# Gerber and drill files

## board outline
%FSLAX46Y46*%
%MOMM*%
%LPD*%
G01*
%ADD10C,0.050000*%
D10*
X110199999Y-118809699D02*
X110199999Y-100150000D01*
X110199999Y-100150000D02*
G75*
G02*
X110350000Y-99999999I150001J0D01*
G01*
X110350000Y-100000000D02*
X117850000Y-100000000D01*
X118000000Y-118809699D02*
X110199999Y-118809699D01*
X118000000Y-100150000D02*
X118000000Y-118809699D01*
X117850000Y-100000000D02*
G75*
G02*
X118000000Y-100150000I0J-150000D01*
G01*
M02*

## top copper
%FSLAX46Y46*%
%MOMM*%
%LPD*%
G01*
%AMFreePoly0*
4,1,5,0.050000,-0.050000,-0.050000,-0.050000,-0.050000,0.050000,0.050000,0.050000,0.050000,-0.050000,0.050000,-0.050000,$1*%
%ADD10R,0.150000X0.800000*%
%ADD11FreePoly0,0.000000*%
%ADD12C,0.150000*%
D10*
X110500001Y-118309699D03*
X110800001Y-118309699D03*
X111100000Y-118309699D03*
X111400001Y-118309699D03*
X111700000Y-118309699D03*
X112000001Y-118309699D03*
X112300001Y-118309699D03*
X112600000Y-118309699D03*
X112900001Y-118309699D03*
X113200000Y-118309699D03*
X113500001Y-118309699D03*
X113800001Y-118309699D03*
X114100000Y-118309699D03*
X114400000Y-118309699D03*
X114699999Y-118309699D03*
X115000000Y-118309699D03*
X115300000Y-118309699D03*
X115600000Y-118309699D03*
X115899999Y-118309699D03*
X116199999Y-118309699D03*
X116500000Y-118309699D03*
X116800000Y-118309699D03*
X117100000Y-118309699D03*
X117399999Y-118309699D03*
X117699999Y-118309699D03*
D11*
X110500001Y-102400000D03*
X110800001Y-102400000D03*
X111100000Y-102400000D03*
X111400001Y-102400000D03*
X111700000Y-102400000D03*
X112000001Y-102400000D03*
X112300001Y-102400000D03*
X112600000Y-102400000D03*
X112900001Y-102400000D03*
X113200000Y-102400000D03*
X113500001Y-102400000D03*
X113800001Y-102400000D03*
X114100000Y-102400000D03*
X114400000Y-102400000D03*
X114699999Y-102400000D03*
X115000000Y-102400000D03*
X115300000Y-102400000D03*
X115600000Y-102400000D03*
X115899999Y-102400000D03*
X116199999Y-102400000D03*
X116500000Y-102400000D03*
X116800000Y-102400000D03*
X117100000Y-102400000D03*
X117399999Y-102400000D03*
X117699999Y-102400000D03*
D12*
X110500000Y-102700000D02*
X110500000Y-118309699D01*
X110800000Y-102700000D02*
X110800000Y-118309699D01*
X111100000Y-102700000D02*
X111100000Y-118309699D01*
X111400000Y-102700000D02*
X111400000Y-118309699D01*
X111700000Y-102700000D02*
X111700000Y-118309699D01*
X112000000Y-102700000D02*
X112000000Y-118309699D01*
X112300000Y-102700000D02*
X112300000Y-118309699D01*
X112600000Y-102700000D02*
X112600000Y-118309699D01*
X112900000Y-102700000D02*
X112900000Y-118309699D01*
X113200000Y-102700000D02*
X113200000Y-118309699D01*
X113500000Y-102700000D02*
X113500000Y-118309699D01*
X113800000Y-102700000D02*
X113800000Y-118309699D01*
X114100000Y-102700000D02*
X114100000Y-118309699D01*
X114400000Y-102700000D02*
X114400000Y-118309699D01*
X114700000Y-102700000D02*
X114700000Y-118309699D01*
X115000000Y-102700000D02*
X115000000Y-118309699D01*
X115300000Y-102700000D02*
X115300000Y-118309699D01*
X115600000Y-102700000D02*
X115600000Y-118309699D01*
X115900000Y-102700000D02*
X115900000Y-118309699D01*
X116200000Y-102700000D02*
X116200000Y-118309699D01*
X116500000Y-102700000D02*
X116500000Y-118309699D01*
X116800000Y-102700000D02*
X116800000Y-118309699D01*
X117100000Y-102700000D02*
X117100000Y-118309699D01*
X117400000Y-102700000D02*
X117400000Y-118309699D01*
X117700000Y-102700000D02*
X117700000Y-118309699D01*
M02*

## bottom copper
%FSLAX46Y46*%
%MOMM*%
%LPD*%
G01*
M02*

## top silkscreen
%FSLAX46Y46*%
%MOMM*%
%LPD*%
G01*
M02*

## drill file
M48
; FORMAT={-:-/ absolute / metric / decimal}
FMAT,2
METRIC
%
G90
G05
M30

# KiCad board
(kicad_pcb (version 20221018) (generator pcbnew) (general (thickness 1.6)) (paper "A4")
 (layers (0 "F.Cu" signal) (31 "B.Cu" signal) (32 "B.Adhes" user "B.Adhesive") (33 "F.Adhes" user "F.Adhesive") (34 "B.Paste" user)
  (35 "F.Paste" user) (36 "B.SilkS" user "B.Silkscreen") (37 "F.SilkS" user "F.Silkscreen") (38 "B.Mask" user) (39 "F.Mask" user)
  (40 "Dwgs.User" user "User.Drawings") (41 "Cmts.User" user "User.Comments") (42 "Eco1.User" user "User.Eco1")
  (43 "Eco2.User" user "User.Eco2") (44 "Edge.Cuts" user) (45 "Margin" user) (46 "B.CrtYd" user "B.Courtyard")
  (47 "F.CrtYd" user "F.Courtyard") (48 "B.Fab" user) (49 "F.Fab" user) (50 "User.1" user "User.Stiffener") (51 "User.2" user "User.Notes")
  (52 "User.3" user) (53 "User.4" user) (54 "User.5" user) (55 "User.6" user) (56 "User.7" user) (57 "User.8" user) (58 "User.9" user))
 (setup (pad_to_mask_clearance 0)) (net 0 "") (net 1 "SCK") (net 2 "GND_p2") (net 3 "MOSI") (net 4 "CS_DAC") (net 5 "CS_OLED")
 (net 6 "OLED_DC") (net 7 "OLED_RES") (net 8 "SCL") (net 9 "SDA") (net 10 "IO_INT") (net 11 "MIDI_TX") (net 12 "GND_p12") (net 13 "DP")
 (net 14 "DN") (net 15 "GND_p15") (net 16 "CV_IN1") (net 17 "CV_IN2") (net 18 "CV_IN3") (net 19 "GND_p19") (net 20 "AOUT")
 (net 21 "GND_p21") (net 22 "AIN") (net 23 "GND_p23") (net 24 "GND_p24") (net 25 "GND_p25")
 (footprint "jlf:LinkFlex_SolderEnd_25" (layer "F.Cu") (at 114.1 118.809699)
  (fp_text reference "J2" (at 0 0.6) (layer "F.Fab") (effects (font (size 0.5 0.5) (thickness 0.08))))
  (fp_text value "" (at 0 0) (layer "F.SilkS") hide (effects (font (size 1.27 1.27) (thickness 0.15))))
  (pad "1" smd rect (at -3.599999 -0.5) (size 0.15 0.8) (layers "F.Cu" "F.Mask") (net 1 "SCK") (thermal_bridge_angle 45))
  (pad "2" smd rect (at -3.299999 -0.5) (size 0.15 0.8) (layers "F.Cu" "F.Mask") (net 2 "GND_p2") (thermal_bridge_angle 45))
  (pad "3" smd rect (at -3 -0.5) (size 0.15 0.8) (layers "F.Cu" "F.Mask") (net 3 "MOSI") (thermal_bridge_angle 45))
  (pad "4" smd rect (at -2.699999 -0.5) (size 0.15 0.8) (layers "F.Cu" "F.Mask") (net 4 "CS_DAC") (thermal_bridge_angle 45))
  (pad "5" smd rect (at -2.4 -0.5) (size 0.15 0.8) (layers "F.Cu" "F.Mask") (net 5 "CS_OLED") (thermal_bridge_angle 45))
  (pad "6" smd rect (at -2.099999 -0.5) (size 0.15 0.8) (layers "F.Cu" "F.Mask") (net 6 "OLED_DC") (thermal_bridge_angle 45))
  (pad "7" smd rect (at -1.799999 -0.5) (size 0.15 0.8) (layers "F.Cu" "F.Mask") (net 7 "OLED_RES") (thermal_bridge_angle 45))
  (pad "8" smd rect (at -1.5 -0.5) (size 0.15 0.8) (layers "F.Cu" "F.Mask") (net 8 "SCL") (thermal_bridge_angle 45))
  (pad "9" smd rect (at -1.199999 -0.5) (size 0.15 0.8) (layers "F.Cu" "F.Mask") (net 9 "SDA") (thermal_bridge_angle 45))
  (pad "10" smd rect (at -0.9 -0.5) (size 0.15 0.8) (layers "F.Cu" "F.Mask") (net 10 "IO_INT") (thermal_bridge_angle 45))
  (pad "11" smd rect (at -0.599999 -0.5) (size 0.15 0.8) (layers "F.Cu" "F.Mask") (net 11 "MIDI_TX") (thermal_bridge_angle 45))
  (pad "12" smd rect (at -0.299999 -0.5) (size 0.15 0.8) (layers "F.Cu" "F.Mask") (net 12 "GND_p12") (thermal_bridge_angle 45))
  (pad "13" smd rect (at 0 -0.5) (size 0.15 0.8) (layers "F.Cu" "F.Mask") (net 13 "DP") (thermal_bridge_angle 45))
  (pad "14" smd rect (at 0.3 -0.5) (size 0.15 0.8) (layers "F.Cu" "F.Mask") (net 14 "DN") (thermal_bridge_angle 45))
  (pad "15" smd rect (at 0.599999 -0.5) (size 0.15 0.8) (layers "F.Cu" "F.Mask") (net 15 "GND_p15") (thermal_bridge_angle 45))
  (pad "16" smd rect (at 0.9 -0.5) (size 0.15 0.8) (layers "F.Cu" "F.Mask") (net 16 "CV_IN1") (thermal_bridge_angle 45))
  (pad "17" smd rect (at 1.2 -0.5) (size 0.15 0.8) (layers "F.Cu" "F.Mask") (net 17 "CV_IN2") (thermal_bridge_angle 45))
  (pad "18" smd rect (at 1.5 -0.5) (size 0.15 0.8) (layers "F.Cu" "F.Mask") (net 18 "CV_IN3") (thermal_bridge_angle 45))
  (pad "19" smd rect (at 1.799999 -0.5) (size 0.15 0.8) (layers "F.Cu" "F.Mask") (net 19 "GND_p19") (thermal_bridge_angle 45))
  (pad "20" smd rect (at 2.099999 -0.5) (size 0.15 0.8) (layers "F.Cu" "F.Mask") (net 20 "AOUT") (thermal_bridge_angle 45))
  (pad "21" smd rect (at 2.4 -0.5) (size 0.15 0.8) (layers "F.Cu" "F.Mask") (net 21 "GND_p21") (thermal_bridge_angle 45))
  (pad "22" smd rect (at 2.7 -0.5) (size 0.15 0.8) (layers "F.Cu" "F.Mask") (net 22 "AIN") (thermal_bridge_angle 45))
  (pad "23" smd rect (at 3 -0.5) (size 0.15 0.8) (layers "F.Cu" "F.Mask") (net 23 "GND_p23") (thermal_bridge_angle 45))
  (pad "24" smd rect (at 3.299999 -0.5) (size 0.15 0.8) (layers "F.Cu" "F.Mask") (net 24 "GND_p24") (thermal_bridge_angle 45))
  (pad "25" smd rect (at 3.599999 -0.5) (size 0.15 0.8) (layers "F.Cu" "F.Mask") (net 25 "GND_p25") (thermal_bridge_angle 45)))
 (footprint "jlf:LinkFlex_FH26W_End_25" (layer "F.Cu") (at 114.1 100)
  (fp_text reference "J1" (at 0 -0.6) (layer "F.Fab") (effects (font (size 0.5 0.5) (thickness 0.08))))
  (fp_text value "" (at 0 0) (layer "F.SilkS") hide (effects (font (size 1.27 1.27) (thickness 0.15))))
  (pad "1" smd custom (at -3.599999 2.4) (size 0.1 0.1) (layers "F.Cu" "F.Mask") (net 1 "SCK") (thermal_bridge_angle 45)
   (options (clearance outline) (anchor rect)) (primitives))
  (pad "2" smd custom (at -3.299999 2.4) (size 0.1 0.1) (layers "F.Cu" "F.Mask") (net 2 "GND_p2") (thermal_bridge_angle 45)
   (options (clearance outline) (anchor rect)) (primitives))
  (pad "3" smd custom (at -3 2.4) (size 0.1 0.1) (layers "F.Cu" "F.Mask") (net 3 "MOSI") (thermal_bridge_angle 45)
   (options (clearance outline) (anchor rect)) (primitives))
  (pad "4" smd custom (at -2.699999 2.4) (size 0.1 0.1) (layers "F.Cu" "F.Mask") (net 4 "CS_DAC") (thermal_bridge_angle 45)
   (options (clearance outline) (anchor rect)) (primitives))
  (pad "5" smd custom (at -2.4 2.4) (size 0.1 0.1) (layers "F.Cu" "F.Mask") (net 5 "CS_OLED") (thermal_bridge_angle 45)
   (options (clearance outline) (anchor rect)) (primitives))
  (pad "6" smd custom (at -2.099999 2.4) (size 0.1 0.1) (layers "F.Cu" "F.Mask") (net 6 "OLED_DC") (thermal_bridge_angle 45)
   (options (clearance outline) (anchor rect)) (primitives))
  (pad "7" smd custom (at -1.799999 2.4) (size 0.1 0.1) (layers "F.Cu" "F.Mask") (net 7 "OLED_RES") (thermal_bridge_angle 45)
   (options (clearance outline) (anchor rect)) (primitives))
  (pad "8" smd custom (at -1.5 2.4) (size 0.1 0.1) (layers "F.Cu" "F.Mask") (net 8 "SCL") (thermal_bridge_angle 45)
   (options (clearance outline) (anchor rect)) (primitives))
  (pad "9" smd custom (at -1.199999 2.4) (size 0.1 0.1) (layers "F.Cu" "F.Mask") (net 9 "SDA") (thermal_bridge_angle 45)
   (options (clearance outline) (anchor rect)) (primitives))
  (pad "10" smd custom (at -0.9 2.4) (size 0.1 0.1) (layers "F.Cu" "F.Mask") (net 10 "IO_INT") (thermal_bridge_angle 45)
   (options (clearance outline) (anchor rect)) (primitives))
  (pad "11" smd custom (at -0.599999 2.4) (size 0.1 0.1) (layers "F.Cu" "F.Mask") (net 11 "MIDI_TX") (thermal_bridge_angle 45)
   (options (clearance outline) (anchor rect)) (primitives))
  (pad "12" smd custom (at -0.299999 2.4) (size 0.1 0.1) (layers "F.Cu" "F.Mask") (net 12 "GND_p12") (thermal_bridge_angle 45)
   (options (clearance outline) (anchor rect)) (primitives))
  (pad "13" smd custom (at 0 2.4) (size 0.1 0.1) (layers "F.Cu" "F.Mask") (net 13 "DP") (thermal_bridge_angle 45)
   (options (clearance outline) (anchor rect)) (primitives))
  (pad "14" smd custom (at 0.3 2.4) (size 0.1 0.1) (layers "F.Cu" "F.Mask") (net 14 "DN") (thermal_bridge_angle 45)
   (options (clearance outline) (anchor rect)) (primitives))
  (pad "15" smd custom (at 0.599999 2.4) (size 0.1 0.1) (layers "F.Cu" "F.Mask") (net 15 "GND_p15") (thermal_bridge_angle 45)
   (options (clearance outline) (anchor rect)) (primitives))
  (pad "16" smd custom (at 0.9 2.4) (size 0.1 0.1) (layers "F.Cu" "F.Mask") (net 16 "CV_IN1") (thermal_bridge_angle 45)
   (options (clearance outline) (anchor rect)) (primitives))
  (pad "17" smd custom (at 1.2 2.4) (size 0.1 0.1) (layers "F.Cu" "F.Mask") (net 17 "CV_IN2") (thermal_bridge_angle 45)
   (options (clearance outline) (anchor rect)) (primitives))
  (pad "18" smd custom (at 1.5 2.4) (size 0.1 0.1) (layers "F.Cu" "F.Mask") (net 18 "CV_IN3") (thermal_bridge_angle 45)
   (options (clearance outline) (anchor rect)) (primitives))
  (pad "19" smd custom (at 1.799999 2.4) (size 0.1 0.1) (layers "F.Cu" "F.Mask") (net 19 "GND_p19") (thermal_bridge_angle 45)
   (options (clearance outline) (anchor rect)) (primitives))
  (pad "20" smd custom (at 2.099999 2.4) (size 0.1 0.1) (layers "F.Cu" "F.Mask") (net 20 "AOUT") (thermal_bridge_angle 45)
   (options (clearance outline) (anchor rect)) (primitives))
  (pad "21" smd custom (at 2.4 2.4) (size 0.1 0.1) (layers "F.Cu" "F.Mask") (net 21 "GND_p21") (thermal_bridge_angle 45)
   (options (clearance outline) (anchor rect)) (primitives))
  (pad "22" smd custom (at 2.7 2.4) (size 0.1 0.1) (layers "F.Cu" "F.Mask") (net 22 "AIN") (thermal_bridge_angle 45)
   (options (clearance outline) (anchor rect)) (primitives))
  (pad "23" smd custom (at 3 2.4) (size 0.1 0.1) (layers "F.Cu" "F.Mask") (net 23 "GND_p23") (thermal_bridge_angle 45)
   (options (clearance outline) (anchor rect)) (primitives))
  (pad "24" smd custom (at 3.299999 2.4) (size 0.1 0.1) (layers "F.Cu" "F.Mask") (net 24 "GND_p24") (thermal_bridge_angle 45)
   (options (clearance outline) (anchor rect)) (primitives))
  (pad "25" smd custom (at 3.599999 2.4) (size 0.1 0.1) (layers "F.Cu" "F.Mask") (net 25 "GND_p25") (thermal_bridge_angle 45)
   (options (clearance outline) (anchor rect)) (primitives)))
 (gr_line (start 110.199999 118.809699) (end 110.199999 100.15) (stroke (width 0.05) (type default)) (layer "Edge.Cuts"))
 (gr_arc (start 110.199999 100.15) (mid 110.243933 100.043933) (end 110.35 99.999999) (stroke (width 0.05) (type default))
  (layer "Edge.Cuts"))
 (gr_line (start 110.35 100) (end 117.85 100) (stroke (width 0.05) (type default)) (layer "Edge.Cuts"))
 (gr_line (start 118 118.809699) (end 110.199999 118.809699) (stroke (width 0.05) (type default)) (layer "Edge.Cuts"))
 (gr_line (start 118 100.15) (end 118 118.809699) (stroke (width 0.05) (type default)) (layer "Edge.Cuts"))
 (gr_arc (start 117.85 100) (mid 117.956066 100.043934) (end 118 100.15) (stroke (width 0.05) (type default)) (layer "Edge.Cuts"))
 (segment (start 110.5 102.7) (end 110.5 118.309699) (width 0.15) (layer "F.Cu") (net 1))
 (segment (start 110.8 102.7) (end 110.8 118.309699) (width 0.15) (layer "F.Cu") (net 2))
 (segment (start 111.1 102.7) (end 111.1 118.309699) (width 0.15) (layer "F.Cu") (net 3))
 (segment (start 111.4 102.7) (end 111.4 118.309699) (width 0.15) (layer "F.Cu") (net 4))
 (segment (start 111.7 102.7) (end 111.7 118.309699) (width 0.15) (layer "F.Cu") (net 5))
 (segment (start 112 102.7) (end 112 118.309699) (width 0.15) (layer "F.Cu") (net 6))
 (segment (start 112.3 102.7) (end 112.3 118.309699) (width 0.15) (layer "F.Cu") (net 7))
 (segment (start 112.6 102.7) (end 112.6 118.309699) (width 0.15) (layer "F.Cu") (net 8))
 (segment (start 112.9 102.7) (end 112.9 118.309699) (width 0.15) (layer "F.Cu") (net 9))
 (segment (start 113.2 102.7) (end 113.2 118.309699) (width 0.15) (layer "F.Cu") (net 10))
 (segment (start 113.5 102.7) (end 113.5 118.309699) (width 0.15) (layer "F.Cu") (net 11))
 (segment (start 113.8 102.7) (end 113.8 118.309699) (width 0.15) (layer "F.Cu") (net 12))
 (segment (start 114.1 102.7) (end 114.1 118.309699) (width 0.15) (layer "F.Cu") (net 13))
 (segment (start 114.4 102.7) (end 114.4 118.309699) (width 0.15) (layer "F.Cu") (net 14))
 (segment (start 114.7 102.7) (end 114.7 118.309699) (width 0.15) (layer "F.Cu") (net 15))
 (segment (start 115 102.7) (end 115 118.309699) (width 0.15) (layer "F.Cu") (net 16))
 (segment (start 115.3 102.7) (end 115.3 118.309699) (width 0.15) (layer "F.Cu") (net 17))
 (segment (start 115.6 102.7) (end 115.6 118.309699) (width 0.15) (layer "F.Cu") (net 18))
 (segment (start 115.9 102.7) (end 115.9 118.309699) (width 0.15) (layer "F.Cu") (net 19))
 (segment (start 116.2 102.7) (end 116.2 118.309699) (width 0.15) (layer "F.Cu") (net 20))
 (segment (start 116.5 102.7) (end 116.5 118.309699) (width 0.15) (layer "F.Cu") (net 21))
 (segment (start 116.8 102.7) (end 116.8 118.309699) (width 0.15) (layer "F.Cu") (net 22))
 (segment (start 117.1 102.7) (end 117.1 118.309699) (width 0.15) (layer "F.Cu") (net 23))
 (segment (start 117.4 102.7) (end 117.4 118.309699) (width 0.15) (layer "F.Cu") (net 24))
 (segment (start 117.7 102.7) (end 117.7 118.309699) (width 0.15) (layer "F.Cu") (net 25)))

